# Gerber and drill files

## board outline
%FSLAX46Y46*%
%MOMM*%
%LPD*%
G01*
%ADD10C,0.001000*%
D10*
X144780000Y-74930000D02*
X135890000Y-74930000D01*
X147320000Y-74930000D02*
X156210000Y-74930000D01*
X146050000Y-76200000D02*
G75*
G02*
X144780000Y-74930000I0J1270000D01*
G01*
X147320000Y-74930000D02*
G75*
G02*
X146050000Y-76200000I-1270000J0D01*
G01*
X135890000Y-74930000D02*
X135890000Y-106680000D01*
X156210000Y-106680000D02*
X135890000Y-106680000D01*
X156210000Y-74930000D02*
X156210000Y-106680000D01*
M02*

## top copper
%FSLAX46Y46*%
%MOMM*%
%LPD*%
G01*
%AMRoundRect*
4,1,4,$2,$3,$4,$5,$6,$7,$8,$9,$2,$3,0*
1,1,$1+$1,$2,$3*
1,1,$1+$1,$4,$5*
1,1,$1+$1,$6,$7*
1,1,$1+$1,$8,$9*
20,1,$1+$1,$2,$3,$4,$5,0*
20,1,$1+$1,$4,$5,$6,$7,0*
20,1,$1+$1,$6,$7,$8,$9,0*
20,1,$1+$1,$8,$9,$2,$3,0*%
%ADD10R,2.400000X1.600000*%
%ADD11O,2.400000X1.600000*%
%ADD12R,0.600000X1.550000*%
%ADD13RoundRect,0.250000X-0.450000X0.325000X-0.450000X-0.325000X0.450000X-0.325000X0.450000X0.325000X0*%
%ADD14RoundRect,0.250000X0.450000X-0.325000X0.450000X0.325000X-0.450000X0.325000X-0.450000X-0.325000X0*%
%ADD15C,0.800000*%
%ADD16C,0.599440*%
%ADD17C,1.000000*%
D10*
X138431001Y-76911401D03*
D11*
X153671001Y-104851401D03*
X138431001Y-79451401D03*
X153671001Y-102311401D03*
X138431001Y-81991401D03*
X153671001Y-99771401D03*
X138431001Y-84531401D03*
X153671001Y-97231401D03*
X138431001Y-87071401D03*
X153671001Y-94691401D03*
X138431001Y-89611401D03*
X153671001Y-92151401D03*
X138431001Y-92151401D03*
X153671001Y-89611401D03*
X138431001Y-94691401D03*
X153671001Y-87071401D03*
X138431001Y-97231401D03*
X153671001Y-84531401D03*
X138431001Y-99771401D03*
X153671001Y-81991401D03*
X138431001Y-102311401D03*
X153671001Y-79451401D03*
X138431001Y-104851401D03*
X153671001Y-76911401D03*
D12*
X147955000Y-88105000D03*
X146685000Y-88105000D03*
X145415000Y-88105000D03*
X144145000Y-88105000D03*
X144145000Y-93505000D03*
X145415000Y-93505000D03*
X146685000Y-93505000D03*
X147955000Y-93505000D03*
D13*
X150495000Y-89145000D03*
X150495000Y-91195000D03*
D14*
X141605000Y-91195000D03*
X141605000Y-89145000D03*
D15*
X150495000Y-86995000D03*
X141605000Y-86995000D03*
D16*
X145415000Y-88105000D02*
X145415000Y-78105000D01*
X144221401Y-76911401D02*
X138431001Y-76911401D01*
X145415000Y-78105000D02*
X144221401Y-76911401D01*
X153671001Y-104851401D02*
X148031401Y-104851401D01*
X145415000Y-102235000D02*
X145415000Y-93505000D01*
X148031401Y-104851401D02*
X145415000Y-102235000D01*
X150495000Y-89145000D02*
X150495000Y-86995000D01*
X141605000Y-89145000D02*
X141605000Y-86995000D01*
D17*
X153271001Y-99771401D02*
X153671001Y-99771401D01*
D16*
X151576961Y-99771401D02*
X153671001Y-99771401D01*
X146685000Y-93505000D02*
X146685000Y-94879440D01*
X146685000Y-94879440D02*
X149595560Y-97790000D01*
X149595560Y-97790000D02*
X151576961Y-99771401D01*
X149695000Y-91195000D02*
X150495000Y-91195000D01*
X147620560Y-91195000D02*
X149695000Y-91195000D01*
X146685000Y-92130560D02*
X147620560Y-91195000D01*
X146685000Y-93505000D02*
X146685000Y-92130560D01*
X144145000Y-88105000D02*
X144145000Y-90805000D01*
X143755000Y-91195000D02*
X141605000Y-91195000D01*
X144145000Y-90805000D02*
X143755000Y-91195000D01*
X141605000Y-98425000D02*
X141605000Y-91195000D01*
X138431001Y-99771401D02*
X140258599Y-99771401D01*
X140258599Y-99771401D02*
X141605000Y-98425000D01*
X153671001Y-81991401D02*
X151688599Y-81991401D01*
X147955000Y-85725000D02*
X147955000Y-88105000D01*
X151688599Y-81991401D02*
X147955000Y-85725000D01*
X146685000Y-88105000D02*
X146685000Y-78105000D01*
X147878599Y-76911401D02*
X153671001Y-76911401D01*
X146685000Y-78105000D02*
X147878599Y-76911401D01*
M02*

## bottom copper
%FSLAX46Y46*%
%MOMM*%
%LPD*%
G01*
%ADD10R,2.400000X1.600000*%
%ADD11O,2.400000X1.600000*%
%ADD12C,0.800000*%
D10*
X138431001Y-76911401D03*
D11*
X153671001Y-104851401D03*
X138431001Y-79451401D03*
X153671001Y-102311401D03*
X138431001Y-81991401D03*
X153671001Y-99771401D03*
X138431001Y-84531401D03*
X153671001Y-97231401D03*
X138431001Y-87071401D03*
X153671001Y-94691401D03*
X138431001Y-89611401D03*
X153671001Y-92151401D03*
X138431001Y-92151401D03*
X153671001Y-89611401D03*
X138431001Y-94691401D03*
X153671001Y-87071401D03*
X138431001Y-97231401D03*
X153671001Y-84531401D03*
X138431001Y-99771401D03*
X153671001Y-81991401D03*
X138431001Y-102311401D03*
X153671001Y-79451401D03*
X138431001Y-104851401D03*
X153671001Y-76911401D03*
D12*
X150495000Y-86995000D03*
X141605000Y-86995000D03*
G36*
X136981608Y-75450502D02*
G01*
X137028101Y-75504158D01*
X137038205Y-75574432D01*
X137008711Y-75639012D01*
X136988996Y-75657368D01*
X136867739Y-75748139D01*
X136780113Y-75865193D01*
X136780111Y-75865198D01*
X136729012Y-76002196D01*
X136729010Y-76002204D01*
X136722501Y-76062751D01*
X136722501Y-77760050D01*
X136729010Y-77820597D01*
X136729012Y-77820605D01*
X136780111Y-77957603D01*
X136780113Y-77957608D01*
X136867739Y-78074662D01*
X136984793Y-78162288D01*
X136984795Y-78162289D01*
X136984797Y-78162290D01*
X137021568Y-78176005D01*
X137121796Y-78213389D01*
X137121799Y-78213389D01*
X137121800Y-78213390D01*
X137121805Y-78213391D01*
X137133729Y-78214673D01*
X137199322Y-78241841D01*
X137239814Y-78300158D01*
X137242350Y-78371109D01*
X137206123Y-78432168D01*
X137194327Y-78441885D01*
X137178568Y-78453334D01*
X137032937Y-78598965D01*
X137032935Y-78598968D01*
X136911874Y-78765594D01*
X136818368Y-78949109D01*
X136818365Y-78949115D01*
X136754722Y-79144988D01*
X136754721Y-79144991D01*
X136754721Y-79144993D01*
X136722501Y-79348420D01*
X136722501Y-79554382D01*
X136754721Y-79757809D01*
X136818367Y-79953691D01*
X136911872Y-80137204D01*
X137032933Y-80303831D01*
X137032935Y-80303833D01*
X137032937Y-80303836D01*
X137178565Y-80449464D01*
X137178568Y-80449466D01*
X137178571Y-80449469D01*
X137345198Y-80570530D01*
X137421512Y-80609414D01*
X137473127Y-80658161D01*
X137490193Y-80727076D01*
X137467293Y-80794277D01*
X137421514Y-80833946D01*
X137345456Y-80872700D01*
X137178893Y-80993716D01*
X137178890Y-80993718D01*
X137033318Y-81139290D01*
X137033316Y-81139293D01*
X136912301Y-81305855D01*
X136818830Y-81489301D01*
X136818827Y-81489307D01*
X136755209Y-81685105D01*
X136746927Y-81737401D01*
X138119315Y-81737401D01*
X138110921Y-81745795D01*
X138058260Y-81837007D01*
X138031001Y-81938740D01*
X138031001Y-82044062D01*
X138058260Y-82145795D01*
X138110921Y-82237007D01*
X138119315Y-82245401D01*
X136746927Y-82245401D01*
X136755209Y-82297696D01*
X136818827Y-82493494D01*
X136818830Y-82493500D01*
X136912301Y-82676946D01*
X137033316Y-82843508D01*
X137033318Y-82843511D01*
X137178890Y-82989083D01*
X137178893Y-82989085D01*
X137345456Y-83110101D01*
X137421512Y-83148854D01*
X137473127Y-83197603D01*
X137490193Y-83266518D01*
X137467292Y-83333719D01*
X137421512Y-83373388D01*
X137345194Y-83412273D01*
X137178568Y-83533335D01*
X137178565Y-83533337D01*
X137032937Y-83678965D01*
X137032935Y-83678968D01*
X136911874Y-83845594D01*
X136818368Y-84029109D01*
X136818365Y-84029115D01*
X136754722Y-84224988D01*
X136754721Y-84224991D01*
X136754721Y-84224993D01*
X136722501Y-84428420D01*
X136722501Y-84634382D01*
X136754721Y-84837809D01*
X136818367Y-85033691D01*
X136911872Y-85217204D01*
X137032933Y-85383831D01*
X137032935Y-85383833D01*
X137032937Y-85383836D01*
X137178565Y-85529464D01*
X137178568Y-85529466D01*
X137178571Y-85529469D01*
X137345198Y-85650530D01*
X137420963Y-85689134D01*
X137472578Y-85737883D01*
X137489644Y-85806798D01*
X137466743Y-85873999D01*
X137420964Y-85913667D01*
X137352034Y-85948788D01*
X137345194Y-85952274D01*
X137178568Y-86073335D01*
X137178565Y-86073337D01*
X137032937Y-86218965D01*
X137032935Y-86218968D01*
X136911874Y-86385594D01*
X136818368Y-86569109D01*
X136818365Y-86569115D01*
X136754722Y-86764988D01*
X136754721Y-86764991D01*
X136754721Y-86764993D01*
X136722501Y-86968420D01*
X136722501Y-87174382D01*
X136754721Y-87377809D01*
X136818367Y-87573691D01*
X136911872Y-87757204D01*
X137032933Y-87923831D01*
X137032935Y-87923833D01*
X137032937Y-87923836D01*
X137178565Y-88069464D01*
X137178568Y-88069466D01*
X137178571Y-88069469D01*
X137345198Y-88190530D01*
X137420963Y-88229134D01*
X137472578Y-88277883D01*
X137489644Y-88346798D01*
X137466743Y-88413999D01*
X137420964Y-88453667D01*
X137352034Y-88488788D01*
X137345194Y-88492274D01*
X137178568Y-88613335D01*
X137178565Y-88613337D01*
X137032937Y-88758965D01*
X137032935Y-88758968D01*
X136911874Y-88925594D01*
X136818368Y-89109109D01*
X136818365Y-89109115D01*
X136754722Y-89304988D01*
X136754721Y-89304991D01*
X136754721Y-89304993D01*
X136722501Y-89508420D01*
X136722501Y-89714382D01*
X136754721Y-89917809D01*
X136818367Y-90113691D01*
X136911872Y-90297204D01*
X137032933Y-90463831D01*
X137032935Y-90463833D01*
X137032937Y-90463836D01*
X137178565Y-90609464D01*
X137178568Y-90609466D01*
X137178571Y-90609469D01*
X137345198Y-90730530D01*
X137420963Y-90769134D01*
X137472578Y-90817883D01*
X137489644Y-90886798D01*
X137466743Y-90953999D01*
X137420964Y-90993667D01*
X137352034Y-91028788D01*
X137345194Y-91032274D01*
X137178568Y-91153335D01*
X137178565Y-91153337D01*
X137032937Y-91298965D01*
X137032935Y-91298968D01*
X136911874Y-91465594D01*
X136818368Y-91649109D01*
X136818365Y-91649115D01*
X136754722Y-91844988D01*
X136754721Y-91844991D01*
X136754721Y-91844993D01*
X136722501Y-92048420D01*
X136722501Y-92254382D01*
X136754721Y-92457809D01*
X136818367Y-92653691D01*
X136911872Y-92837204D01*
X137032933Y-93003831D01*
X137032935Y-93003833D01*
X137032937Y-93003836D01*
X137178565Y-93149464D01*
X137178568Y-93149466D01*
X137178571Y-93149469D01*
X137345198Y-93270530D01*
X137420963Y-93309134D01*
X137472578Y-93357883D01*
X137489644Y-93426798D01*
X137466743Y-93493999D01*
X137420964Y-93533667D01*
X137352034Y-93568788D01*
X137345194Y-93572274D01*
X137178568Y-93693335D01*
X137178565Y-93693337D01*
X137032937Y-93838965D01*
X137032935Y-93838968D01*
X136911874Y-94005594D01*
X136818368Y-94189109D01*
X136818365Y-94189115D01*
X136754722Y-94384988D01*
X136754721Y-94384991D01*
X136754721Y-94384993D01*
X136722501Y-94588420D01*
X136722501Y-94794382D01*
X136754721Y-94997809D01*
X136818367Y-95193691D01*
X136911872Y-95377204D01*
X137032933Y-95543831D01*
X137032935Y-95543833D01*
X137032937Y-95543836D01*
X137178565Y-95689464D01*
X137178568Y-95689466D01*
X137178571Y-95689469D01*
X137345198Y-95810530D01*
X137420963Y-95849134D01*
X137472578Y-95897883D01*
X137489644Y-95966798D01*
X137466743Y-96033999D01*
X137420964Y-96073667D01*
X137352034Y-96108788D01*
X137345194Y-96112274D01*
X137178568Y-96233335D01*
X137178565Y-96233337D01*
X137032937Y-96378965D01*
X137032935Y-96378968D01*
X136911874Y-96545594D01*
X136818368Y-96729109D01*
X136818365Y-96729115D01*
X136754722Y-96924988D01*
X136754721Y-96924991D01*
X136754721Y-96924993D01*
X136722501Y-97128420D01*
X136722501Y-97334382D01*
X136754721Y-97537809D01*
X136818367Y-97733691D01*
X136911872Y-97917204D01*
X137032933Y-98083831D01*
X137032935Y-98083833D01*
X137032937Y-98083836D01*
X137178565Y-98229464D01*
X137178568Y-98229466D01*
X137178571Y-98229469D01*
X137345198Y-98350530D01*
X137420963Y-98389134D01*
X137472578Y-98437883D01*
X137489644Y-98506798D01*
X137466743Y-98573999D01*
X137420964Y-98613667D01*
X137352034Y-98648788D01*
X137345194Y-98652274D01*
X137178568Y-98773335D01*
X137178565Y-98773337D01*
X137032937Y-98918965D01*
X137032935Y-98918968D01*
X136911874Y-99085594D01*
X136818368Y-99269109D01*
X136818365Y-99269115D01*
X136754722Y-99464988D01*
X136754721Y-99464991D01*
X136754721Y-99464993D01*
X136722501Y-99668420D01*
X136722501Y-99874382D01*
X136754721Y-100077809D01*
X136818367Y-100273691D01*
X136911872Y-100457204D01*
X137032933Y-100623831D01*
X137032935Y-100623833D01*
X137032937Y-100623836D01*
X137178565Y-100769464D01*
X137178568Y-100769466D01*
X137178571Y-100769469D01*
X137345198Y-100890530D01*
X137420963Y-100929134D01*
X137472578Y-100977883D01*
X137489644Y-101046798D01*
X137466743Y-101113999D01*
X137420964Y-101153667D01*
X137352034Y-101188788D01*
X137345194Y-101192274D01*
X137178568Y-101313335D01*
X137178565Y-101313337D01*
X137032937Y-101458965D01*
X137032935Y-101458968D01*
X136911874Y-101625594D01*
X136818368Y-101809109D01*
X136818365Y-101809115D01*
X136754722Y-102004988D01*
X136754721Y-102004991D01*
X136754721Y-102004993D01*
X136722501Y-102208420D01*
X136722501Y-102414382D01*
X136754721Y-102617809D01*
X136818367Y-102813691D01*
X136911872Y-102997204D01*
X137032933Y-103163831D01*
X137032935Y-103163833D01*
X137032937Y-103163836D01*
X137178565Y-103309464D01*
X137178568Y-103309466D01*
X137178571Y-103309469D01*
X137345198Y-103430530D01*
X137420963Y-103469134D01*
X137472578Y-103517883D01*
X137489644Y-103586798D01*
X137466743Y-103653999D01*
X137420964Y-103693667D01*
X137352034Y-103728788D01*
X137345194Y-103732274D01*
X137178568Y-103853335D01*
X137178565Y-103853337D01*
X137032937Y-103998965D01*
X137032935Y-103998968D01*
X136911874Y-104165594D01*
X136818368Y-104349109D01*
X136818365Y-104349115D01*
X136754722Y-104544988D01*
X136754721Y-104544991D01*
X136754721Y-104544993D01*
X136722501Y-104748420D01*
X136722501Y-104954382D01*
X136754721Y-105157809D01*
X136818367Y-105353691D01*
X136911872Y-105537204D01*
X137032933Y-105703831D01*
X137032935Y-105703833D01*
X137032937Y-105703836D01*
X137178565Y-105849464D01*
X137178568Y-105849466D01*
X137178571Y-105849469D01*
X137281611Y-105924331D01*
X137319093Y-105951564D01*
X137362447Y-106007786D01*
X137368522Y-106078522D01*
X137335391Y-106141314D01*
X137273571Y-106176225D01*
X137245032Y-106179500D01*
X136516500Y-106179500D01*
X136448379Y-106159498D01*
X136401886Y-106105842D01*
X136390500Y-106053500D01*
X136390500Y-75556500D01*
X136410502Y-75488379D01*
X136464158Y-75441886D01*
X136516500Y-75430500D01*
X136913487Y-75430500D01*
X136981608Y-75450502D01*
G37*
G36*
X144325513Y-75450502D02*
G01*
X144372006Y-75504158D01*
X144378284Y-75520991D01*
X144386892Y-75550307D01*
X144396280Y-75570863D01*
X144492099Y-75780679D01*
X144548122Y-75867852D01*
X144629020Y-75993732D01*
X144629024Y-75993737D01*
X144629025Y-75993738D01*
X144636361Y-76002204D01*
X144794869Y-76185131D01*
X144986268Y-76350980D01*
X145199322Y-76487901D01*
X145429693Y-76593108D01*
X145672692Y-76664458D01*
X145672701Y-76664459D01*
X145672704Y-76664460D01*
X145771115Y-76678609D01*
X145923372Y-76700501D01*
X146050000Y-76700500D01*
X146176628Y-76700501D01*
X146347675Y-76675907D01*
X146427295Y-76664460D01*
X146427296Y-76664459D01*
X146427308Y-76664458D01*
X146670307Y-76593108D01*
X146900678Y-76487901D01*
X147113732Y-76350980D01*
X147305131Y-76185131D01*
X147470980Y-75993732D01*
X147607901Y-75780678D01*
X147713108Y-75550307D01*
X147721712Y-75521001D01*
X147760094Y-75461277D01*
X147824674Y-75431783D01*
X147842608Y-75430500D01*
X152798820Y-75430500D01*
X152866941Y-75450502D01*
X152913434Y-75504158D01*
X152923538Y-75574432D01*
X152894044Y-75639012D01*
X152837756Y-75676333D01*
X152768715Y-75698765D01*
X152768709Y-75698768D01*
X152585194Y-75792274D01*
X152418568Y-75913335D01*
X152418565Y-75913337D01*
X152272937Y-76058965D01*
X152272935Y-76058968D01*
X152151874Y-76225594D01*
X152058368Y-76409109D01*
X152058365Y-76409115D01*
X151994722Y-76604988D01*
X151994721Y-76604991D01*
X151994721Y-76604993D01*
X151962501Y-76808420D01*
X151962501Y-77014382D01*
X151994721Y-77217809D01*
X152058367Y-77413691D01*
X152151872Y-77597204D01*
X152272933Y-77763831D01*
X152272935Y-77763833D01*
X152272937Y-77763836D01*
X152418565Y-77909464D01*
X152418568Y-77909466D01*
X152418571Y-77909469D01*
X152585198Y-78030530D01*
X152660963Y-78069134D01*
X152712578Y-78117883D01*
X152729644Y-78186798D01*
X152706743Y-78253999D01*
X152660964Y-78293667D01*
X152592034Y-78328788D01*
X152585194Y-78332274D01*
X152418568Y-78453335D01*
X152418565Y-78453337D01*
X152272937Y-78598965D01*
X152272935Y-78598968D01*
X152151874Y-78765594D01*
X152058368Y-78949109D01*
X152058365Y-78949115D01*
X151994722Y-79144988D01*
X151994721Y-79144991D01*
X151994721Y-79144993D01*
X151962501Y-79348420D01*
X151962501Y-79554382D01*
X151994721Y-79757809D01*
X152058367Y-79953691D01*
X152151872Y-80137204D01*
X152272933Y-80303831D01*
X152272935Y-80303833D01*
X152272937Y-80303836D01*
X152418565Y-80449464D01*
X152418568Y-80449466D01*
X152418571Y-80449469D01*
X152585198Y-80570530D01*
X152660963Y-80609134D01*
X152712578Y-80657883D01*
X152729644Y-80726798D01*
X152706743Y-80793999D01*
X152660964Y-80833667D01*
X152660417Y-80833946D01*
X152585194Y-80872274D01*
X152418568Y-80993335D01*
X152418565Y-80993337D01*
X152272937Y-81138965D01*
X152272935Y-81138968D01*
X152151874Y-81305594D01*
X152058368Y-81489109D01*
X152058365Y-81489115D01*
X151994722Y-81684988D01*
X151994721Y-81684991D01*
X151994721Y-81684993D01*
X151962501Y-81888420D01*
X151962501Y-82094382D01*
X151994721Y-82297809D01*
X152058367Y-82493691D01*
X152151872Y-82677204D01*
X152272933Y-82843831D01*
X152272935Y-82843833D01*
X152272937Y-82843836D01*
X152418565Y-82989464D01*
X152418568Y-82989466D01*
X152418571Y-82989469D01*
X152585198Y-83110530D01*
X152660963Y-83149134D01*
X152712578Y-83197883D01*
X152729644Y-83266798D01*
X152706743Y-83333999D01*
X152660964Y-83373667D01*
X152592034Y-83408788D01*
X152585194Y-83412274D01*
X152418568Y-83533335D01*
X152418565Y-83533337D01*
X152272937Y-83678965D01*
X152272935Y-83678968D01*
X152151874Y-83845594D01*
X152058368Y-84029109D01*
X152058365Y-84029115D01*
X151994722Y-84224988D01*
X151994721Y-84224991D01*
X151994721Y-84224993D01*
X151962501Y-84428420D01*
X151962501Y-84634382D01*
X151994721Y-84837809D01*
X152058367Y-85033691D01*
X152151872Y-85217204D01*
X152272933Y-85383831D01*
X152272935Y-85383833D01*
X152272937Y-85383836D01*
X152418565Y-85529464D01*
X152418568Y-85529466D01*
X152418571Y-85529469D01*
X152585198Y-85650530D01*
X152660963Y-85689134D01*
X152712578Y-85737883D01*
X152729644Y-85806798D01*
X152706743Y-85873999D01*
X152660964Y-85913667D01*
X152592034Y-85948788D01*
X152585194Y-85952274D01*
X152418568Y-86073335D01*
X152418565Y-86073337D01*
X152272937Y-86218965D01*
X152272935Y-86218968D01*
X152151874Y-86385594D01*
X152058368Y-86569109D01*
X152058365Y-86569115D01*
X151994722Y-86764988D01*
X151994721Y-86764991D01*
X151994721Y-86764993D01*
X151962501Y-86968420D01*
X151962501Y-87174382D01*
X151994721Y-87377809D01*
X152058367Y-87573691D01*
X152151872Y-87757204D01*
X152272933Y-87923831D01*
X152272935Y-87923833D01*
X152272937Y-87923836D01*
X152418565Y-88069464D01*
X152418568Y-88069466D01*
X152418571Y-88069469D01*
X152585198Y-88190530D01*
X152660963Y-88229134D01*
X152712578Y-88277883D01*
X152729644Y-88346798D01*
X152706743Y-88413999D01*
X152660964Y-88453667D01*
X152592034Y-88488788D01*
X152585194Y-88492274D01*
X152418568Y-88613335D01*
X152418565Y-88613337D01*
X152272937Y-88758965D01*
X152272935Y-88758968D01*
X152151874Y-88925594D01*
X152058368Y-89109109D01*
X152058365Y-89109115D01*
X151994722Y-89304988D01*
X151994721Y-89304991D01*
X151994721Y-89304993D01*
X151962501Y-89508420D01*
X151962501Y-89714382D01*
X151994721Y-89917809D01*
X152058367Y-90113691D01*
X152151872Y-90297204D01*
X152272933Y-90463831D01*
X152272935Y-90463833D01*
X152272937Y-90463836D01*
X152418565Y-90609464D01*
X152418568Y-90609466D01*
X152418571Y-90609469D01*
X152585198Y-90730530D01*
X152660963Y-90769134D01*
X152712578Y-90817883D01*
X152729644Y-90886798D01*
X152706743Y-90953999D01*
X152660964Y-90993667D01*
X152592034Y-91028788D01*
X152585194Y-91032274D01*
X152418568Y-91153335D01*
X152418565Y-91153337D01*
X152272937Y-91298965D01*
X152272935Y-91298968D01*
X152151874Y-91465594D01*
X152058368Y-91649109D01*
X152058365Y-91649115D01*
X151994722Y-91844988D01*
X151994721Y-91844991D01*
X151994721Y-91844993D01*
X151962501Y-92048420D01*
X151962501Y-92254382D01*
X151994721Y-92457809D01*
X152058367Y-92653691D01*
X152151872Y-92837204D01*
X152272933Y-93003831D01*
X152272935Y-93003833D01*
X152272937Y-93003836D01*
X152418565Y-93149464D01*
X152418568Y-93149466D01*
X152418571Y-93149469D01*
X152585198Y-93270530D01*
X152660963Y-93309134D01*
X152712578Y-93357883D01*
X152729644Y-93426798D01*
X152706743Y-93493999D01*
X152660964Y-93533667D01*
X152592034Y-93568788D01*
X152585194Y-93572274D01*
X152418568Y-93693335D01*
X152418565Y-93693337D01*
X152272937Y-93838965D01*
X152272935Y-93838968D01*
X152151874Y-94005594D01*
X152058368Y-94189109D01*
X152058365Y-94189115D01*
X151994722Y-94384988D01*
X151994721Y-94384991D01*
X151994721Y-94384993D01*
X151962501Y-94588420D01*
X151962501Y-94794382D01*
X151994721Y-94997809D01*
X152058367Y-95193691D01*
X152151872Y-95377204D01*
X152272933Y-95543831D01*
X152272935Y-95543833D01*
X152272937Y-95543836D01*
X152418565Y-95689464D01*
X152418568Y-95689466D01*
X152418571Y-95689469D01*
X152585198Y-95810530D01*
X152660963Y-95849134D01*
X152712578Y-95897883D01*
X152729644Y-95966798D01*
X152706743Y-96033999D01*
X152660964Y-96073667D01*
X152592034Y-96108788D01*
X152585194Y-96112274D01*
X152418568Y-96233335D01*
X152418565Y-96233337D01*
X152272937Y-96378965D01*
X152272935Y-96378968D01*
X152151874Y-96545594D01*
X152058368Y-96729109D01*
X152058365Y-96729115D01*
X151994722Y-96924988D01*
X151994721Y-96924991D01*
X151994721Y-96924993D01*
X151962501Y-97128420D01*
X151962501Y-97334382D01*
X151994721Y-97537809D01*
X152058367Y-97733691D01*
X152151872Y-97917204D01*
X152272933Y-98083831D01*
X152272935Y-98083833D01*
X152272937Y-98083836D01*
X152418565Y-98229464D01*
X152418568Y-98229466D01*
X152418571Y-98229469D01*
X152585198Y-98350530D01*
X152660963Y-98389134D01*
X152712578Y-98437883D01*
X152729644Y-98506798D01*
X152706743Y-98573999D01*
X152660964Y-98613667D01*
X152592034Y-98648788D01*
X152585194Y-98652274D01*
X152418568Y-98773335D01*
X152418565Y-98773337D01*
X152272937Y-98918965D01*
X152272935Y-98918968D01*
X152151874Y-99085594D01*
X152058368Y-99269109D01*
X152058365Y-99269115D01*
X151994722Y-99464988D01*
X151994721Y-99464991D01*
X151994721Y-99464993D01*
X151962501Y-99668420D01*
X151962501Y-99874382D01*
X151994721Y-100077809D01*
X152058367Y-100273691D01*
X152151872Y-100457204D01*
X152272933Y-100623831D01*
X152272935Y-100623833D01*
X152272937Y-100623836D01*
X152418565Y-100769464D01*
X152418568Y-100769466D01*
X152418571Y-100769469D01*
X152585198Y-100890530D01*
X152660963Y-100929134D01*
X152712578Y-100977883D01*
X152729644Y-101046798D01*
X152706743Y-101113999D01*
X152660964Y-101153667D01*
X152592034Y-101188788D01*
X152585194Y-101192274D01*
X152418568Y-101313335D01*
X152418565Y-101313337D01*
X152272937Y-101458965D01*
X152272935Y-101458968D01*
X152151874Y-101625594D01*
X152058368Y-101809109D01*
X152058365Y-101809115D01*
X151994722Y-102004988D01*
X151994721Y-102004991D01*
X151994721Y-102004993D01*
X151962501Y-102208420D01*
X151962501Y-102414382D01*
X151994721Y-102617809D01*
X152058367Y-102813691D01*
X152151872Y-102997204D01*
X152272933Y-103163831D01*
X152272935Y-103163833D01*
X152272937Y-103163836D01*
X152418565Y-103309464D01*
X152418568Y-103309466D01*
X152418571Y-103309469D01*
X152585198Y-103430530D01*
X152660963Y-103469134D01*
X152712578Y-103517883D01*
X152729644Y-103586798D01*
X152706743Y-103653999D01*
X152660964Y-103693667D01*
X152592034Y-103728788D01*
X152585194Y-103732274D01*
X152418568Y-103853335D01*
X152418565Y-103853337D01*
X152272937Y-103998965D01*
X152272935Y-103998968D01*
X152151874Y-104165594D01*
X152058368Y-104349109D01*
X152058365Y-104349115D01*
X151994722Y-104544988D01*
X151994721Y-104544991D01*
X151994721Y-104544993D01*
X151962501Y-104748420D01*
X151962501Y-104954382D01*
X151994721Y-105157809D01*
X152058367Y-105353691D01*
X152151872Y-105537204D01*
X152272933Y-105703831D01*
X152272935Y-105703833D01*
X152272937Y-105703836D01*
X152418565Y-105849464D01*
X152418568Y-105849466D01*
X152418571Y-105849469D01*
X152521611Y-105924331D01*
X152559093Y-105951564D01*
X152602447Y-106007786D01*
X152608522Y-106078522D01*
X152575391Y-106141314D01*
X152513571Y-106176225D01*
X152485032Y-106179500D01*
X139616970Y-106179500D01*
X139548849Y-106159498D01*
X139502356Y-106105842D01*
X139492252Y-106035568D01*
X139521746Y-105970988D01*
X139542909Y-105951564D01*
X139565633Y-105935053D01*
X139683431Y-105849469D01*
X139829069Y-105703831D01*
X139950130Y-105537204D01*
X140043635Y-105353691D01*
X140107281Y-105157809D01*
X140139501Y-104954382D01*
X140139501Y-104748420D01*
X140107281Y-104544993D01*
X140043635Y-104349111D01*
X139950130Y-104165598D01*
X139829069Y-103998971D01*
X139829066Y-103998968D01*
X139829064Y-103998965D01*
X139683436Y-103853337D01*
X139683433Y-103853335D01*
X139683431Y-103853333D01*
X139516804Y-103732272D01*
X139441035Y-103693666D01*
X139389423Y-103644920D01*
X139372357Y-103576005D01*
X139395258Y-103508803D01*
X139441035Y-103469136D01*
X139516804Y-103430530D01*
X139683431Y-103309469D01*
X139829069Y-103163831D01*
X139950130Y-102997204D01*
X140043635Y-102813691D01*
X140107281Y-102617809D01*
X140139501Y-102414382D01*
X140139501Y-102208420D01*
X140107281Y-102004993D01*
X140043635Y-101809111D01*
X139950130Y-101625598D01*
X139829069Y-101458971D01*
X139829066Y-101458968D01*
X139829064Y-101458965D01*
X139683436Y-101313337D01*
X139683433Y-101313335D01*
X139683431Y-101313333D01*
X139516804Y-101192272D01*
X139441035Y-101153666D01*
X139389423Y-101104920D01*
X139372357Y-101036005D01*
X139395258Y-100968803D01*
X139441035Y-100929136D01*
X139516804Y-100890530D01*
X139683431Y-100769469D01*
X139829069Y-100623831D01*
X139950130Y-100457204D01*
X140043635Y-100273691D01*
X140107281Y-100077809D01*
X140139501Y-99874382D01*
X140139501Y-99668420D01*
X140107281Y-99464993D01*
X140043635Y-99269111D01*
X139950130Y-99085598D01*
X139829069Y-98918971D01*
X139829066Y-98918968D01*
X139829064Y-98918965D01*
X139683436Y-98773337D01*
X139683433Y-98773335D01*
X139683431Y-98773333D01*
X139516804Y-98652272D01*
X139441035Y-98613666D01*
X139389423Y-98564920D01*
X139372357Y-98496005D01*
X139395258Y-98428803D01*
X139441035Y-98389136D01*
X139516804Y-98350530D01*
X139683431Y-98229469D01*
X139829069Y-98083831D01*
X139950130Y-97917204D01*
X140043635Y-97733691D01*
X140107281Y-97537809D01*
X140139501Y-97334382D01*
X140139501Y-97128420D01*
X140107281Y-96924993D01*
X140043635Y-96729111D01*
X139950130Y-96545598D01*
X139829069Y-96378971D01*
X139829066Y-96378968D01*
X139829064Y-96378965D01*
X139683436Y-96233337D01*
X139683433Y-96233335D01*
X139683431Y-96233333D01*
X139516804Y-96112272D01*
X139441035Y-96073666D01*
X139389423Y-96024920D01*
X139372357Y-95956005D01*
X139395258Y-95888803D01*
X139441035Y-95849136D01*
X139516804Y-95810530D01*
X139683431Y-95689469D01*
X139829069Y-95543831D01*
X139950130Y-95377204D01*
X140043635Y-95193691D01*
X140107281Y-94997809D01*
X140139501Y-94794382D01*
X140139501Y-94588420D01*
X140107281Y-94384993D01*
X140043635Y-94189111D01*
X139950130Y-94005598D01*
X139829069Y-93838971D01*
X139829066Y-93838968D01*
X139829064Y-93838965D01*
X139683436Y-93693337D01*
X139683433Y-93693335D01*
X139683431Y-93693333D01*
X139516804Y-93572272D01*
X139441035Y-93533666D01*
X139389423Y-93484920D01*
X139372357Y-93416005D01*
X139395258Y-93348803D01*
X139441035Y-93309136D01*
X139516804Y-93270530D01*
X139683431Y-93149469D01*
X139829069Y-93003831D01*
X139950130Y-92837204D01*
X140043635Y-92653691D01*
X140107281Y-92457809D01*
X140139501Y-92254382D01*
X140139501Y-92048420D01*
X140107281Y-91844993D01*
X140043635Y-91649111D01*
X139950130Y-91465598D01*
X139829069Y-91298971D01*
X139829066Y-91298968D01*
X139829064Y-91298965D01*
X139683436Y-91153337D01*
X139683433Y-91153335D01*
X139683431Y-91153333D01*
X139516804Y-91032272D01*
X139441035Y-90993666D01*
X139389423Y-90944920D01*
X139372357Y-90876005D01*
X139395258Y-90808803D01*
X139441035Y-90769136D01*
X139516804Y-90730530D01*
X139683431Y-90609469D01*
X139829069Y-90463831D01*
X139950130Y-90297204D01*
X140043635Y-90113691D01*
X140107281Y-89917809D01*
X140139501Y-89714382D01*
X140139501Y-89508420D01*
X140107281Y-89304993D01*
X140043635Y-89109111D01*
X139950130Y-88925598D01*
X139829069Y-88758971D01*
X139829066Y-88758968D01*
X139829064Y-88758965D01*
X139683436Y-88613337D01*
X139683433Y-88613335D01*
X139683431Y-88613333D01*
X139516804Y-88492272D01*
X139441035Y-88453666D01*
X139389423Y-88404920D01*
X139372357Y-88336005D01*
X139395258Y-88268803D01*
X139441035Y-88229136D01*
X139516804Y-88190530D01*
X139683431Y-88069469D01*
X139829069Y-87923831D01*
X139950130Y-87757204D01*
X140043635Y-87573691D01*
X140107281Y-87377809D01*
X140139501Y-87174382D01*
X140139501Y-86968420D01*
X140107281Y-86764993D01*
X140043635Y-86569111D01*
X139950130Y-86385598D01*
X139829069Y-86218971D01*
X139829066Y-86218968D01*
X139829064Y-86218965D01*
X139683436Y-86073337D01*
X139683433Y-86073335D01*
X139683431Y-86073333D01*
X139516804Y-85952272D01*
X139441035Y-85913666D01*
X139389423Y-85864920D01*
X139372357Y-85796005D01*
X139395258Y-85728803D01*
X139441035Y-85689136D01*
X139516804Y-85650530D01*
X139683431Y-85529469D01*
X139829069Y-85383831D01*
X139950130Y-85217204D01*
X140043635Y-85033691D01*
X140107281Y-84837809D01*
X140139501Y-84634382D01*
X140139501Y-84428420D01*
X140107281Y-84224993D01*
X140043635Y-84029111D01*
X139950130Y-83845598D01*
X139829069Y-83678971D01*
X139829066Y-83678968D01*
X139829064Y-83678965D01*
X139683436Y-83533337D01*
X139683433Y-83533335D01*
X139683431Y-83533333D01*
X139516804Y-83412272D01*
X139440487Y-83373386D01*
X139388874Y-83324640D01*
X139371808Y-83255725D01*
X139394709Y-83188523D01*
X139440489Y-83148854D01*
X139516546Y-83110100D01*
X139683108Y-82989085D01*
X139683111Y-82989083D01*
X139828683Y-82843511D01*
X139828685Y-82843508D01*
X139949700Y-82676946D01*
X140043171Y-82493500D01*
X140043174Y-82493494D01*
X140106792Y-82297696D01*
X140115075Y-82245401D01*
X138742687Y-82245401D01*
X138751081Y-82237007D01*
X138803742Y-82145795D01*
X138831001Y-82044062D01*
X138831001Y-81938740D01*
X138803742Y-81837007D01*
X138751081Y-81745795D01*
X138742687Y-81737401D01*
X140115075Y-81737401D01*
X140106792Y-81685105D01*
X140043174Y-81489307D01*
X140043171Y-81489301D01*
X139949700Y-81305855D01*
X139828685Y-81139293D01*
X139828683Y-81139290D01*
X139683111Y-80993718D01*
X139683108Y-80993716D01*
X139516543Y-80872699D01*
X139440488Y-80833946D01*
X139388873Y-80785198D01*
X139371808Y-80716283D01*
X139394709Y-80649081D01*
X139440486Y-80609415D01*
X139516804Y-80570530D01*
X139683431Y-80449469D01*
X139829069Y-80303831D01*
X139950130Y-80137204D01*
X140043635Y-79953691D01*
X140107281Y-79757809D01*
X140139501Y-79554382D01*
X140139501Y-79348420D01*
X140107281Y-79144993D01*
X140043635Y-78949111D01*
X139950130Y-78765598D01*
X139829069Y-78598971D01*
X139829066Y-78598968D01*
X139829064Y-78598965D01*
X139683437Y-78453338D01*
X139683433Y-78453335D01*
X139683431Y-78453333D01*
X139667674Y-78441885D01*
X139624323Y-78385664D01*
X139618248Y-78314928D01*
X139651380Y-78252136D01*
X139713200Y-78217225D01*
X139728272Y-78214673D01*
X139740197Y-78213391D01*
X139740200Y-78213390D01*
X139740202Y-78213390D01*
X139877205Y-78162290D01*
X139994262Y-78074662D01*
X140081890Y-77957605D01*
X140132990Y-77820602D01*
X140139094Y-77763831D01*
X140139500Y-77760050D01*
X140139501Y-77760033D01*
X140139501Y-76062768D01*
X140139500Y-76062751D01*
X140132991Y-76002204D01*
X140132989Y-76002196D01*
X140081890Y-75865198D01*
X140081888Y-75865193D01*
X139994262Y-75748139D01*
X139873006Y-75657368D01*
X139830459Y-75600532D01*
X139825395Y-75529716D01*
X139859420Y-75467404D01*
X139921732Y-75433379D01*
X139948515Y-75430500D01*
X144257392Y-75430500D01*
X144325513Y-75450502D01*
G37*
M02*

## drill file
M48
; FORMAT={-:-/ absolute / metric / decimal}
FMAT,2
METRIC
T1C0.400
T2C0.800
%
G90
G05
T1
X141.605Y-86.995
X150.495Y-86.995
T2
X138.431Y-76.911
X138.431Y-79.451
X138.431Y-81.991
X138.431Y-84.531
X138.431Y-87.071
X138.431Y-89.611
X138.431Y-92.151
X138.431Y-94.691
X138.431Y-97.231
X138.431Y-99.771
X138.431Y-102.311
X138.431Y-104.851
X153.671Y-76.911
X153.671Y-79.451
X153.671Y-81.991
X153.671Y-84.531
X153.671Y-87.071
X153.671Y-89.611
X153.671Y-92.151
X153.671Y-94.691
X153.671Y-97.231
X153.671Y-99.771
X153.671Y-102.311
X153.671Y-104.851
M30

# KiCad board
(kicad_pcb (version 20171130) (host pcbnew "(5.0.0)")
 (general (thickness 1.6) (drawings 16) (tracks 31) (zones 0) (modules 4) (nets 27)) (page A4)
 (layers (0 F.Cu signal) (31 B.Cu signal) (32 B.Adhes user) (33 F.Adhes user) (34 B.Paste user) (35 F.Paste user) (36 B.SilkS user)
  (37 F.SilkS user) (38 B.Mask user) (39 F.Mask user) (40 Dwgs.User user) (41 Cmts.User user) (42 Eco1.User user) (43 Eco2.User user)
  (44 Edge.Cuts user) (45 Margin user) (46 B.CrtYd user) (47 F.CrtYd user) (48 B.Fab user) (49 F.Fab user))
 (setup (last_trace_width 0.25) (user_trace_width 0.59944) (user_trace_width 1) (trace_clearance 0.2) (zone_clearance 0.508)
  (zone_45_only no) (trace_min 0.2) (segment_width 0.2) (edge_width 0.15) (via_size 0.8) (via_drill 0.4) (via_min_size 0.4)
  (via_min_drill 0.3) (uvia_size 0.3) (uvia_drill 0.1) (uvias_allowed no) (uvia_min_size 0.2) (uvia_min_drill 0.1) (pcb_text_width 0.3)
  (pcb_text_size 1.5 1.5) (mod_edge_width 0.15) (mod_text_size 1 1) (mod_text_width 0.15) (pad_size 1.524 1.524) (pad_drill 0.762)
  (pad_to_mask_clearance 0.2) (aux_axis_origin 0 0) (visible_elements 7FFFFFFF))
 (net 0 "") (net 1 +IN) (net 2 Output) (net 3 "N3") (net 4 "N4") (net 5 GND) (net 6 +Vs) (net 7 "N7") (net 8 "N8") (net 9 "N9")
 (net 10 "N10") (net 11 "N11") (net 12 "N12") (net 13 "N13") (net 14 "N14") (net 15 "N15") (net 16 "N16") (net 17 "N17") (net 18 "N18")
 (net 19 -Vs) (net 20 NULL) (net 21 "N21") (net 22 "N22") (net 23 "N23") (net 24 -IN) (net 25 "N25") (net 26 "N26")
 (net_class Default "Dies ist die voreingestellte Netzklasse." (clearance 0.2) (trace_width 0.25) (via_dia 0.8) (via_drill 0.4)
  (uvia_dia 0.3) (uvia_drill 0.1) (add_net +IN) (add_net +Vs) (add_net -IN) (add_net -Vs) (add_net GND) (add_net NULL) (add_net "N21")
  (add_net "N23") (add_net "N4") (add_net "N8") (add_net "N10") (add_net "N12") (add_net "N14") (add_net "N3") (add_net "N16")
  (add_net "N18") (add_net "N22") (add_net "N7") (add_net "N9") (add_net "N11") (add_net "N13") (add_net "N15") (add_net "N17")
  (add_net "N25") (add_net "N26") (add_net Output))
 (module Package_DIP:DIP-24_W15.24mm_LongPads (layer F.Cu) (at 138.431001 76.911401)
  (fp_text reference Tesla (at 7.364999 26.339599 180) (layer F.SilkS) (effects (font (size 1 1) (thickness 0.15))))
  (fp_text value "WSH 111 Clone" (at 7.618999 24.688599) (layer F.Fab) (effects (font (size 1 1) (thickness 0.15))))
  (pad 1 thru_hole rect (at 0 0) (size 2.4 1.6) (drill 0.8) (layers *.Cu *.Mask) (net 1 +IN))
  (pad 13 thru_hole oval (at 15.24 27.94) (size 2.4 1.6) (drill 0.8) (layers *.Cu *.Mask) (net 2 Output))
  (pad 2 thru_hole oval (at 0 2.54) (size 2.4 1.6) (drill 0.8) (layers *.Cu *.Mask) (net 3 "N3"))
  (pad 14 thru_hole oval (at 15.24 25.4) (size 2.4 1.6) (drill 0.8) (layers *.Cu *.Mask) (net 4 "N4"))
  (pad 3 thru_hole oval (at 0 5.08) (size 2.4 1.6) (drill 0.8) (layers *.Cu *.Mask) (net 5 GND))
  (pad 15 thru_hole oval (at 15.24 22.86) (size 2.4 1.6) (drill 0.8) (layers *.Cu *.Mask) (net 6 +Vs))
  (pad 4 thru_hole oval (at 0 7.62) (size 2.4 1.6) (drill 0.8) (layers *.Cu *.Mask) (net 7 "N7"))
  (pad 16 thru_hole oval (at 15.24 20.32) (size 2.4 1.6) (drill 0.8) (layers *.Cu *.Mask) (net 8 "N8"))
  (pad 5 thru_hole oval (at 0 10.16) (size 2.4 1.6) (drill 0.8) (layers *.Cu *.Mask) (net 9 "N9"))
  (pad 17 thru_hole oval (at 15.24 17.78) (size 2.4 1.6) (drill 0.8) (layers *.Cu *.Mask) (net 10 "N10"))
  (pad 6 thru_hole oval (at 0 12.7) (size 2.4 1.6) (drill 0.8) (layers *.Cu *.Mask) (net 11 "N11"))
  (pad 18 thru_hole oval (at 15.24 15.24) (size 2.4 1.6) (drill 0.8) (layers *.Cu *.Mask) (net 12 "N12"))
  (pad 7 thru_hole oval (at 0 15.24) (size 2.4 1.6) (drill 0.8) (layers *.Cu *.Mask) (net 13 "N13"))
  (pad 19 thru_hole oval (at 15.24 12.7) (size 2.4 1.6) (drill 0.8) (layers *.Cu *.Mask) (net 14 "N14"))
  (pad 8 thru_hole oval (at 0 17.78) (size 2.4 1.6) (drill 0.8) (layers *.Cu *.Mask) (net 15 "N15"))
  (pad 20 thru_hole oval (at 15.24 10.16) (size 2.4 1.6) (drill 0.8) (layers *.Cu *.Mask) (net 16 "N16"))
  (pad 9 thru_hole oval (at 0 20.32) (size 2.4 1.6) (drill 0.8) (layers *.Cu *.Mask) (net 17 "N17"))
  (pad 21 thru_hole oval (at 15.24 7.62) (size 2.4 1.6) (drill 0.8) (layers *.Cu *.Mask) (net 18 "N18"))
  (pad 10 thru_hole oval (at 0 22.86) (size 2.4 1.6) (drill 0.8) (layers *.Cu *.Mask) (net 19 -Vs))
  (pad 22 thru_hole oval (at 15.24 5.08) (size 2.4 1.6) (drill 0.8) (layers *.Cu *.Mask) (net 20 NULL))
  (pad 11 thru_hole oval (at 0 25.4) (size 2.4 1.6) (drill 0.8) (layers *.Cu *.Mask) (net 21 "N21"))
  (pad 23 thru_hole oval (at 15.24 2.54) (size 2.4 1.6) (drill 0.8) (layers *.Cu *.Mask) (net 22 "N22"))
  (pad 12 thru_hole oval (at 0 27.94) (size 2.4 1.6) (drill 0.8) (layers *.Cu *.Mask) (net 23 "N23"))
  (pad 24 thru_hole oval (at 15.24 0) (size 2.4 1.6) (drill 0.8) (layers *.Cu *.Mask) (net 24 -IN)))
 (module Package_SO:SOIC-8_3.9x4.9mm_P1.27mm (layer F.Cu) (at 146.05 90.805 270)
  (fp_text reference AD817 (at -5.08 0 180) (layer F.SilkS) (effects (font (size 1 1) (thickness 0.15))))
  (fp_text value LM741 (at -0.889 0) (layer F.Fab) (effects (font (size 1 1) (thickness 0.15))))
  (pad 1 smd rect (at -2.7 -1.905 270) (size 1.55 0.6) (layers F.Cu F.Paste F.Mask) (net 20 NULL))
  (pad 2 smd rect (at -2.7 -0.635 270) (size 1.55 0.6) (layers F.Cu F.Paste F.Mask) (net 24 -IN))
  (pad 3 smd rect (at -2.7 0.635 270) (size 1.55 0.6) (layers F.Cu F.Paste F.Mask) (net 1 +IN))
  (pad 4 smd rect (at -2.7 1.905 270) (size 1.55 0.6) (layers F.Cu F.Paste F.Mask) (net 19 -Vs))
  (pad 5 smd rect (at 2.7 1.905 270) (size 1.55 0.6) (layers F.Cu F.Paste F.Mask) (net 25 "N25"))
  (pad 6 smd rect (at 2.7 0.635 270) (size 1.55 0.6) (layers F.Cu F.Paste F.Mask) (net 2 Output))
  (pad 7 smd rect (at 2.7 -0.635 270) (size 1.55 0.6) (layers F.Cu F.Paste F.Mask) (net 6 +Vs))
  (pad 8 smd rect (at 2.7 -1.905 270) (size 1.55 0.6) (layers F.Cu F.Paste F.Mask) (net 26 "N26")))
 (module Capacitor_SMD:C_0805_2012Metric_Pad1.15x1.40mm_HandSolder (layer F.Cu) (at 150.495 90.17 270)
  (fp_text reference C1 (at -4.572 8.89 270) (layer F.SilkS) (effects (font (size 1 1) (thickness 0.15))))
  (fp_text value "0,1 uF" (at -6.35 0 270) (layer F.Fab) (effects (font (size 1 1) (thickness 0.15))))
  (pad 1 smd roundrect (at -1.025 0 270) (size 1.15 1.4) (layers F.Cu F.Paste F.Mask) (roundrect_rratio 0.217391) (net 5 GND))
  (pad 2 smd roundrect (at 1.025 0 270) (size 1.15 1.4) (layers F.Cu F.Paste F.Mask) (roundrect_rratio 0.217391) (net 6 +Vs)))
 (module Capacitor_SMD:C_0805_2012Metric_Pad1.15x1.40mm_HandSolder (layer F.Cu) (at 141.605 90.17 90)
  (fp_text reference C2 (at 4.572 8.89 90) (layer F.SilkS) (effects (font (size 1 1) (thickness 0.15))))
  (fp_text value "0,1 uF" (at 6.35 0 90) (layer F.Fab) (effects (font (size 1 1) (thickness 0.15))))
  (pad 1 smd roundrect (at -1.025 0 90) (size 1.15 1.4) (layers F.Cu F.Paste F.Mask) (roundrect_rratio 0.217391) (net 19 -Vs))
  (pad 2 smd roundrect (at 1.025 0 90) (size 1.15 1.4) (layers F.Cu F.Paste F.Mask) (roundrect_rratio 0.217391) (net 5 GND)))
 (gr_line (start 144.78 74.93) (end 135.89 74.93) (layer Edge.Cuts) (width 0.001))
 (gr_line (start 147.32 74.93) (end 156.21 74.93) (layer Edge.Cuts) (width 0.001))
 (gr_arc (start 146.05 74.93) (end 144.78 74.93) (angle -90) (layer Edge.Cuts) (width 0.001))
 (gr_arc (start 146.05 74.93) (end 146.05 76.2) (angle -90) (layer Edge.Cuts) (width 0.001))
 (gr_line (start 135.89 74.93) (end 135.89 106.68) (layer Edge.Cuts) (width 0.001))
 (gr_line (start 156.21 106.68) (end 135.89 106.68) (layer Edge.Cuts) (width 0.001))
 (gr_line (start 156.21 74.93) (end 156.21 106.68) (layer Edge.Cuts) (width 0.001))
 (segment (start 145.415 88.105) (end 145.415 78.105) (width 0.59944) (layer F.Cu) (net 1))
 (segment (start 144.221401 76.911401) (end 138.431001 76.911401) (width 0.59944) (layer F.Cu) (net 1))
 (segment (start 145.415 78.105) (end 144.221401 76.911401) (width 0.59944) (layer F.Cu) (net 1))
 (segment (start 153.671001 104.851401) (end 148.031401 104.851401) (width 0.59944) (layer F.Cu) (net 2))
 (segment (start 145.415 102.235) (end 145.415 93.505) (width 0.59944) (layer F.Cu) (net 2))
 (segment (start 148.031401 104.851401) (end 145.415 102.235) (width 0.59944) (layer F.Cu) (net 2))
 (segment (start 150.495 89.145) (end 150.495 86.995) (width 0.59944) (layer F.Cu) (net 5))
 (via (at 150.495 86.995) (size 0.8) (drill 0.4) (layers F.Cu B.Cu) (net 5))
 (segment (start 141.605 89.145) (end 141.605 86.995) (width 0.59944) (layer F.Cu) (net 5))
 (via (at 141.605 86.995) (size 0.8) (drill 0.4) (layers F.Cu B.Cu) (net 5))
 (segment (start 153.271001 99.771401) (end 153.671001 99.771401) (width 1) (layer F.Cu) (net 6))
 (segment (start 151.576961 99.771401) (end 153.671001 99.771401) (width 0.59944) (layer F.Cu) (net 6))
 (segment (start 146.685 93.505) (end 146.685 94.87944) (width 0.59944) (layer F.Cu) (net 6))
 (segment (start 146.685 94.87944) (end 149.59556 97.79) (width 0.59944) (layer F.Cu) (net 6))
 (segment (start 149.59556 97.79) (end 151.576961 99.771401) (width 0.59944) (layer F.Cu) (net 6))
 (segment (start 149.695 91.195) (end 150.495 91.195) (width 0.59944) (layer F.Cu) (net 6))
 (segment (start 147.62056 91.195) (end 149.695 91.195) (width 0.59944) (layer F.Cu) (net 6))
 (segment (start 146.685 92.13056) (end 147.62056 91.195) (width 0.59944) (layer F.Cu) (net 6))
 (segment (start 146.685 93.505) (end 146.685 92.13056) (width 0.59944) (layer F.Cu) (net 6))
 (segment (start 144.145 88.105) (end 144.145 90.805) (width 0.59944) (layer F.Cu) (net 19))
 (segment (start 143.755 91.195) (end 141.605 91.195) (width 0.59944) (layer F.Cu) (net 19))
 (segment (start 144.145 90.805) (end 143.755 91.195) (width 0.59944) (layer F.Cu) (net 19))
 (segment (start 141.605 98.425) (end 141.605 91.195) (width 0.59944) (layer F.Cu) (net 19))
 (segment (start 138.431001 99.771401) (end 140.258599 99.771401) (width 0.59944) (layer F.Cu) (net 19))
 (segment (start 140.258599 99.771401) (end 141.605 98.425) (width 0.59944) (layer F.Cu) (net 19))
 (segment (start 153.671001 81.991401) (end 151.688599 81.991401) (width 0.59944) (layer F.Cu) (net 20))
 (segment (start 147.955 85.725) (end 147.955 88.105) (width 0.59944) (layer F.Cu) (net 20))
 (segment (start 151.688599 81.991401) (end 147.955 85.725) (width 0.59944) (layer F.Cu) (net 20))
 (segment (start 146.685 88.105) (end 146.685 78.105) (width 0.59944) (layer F.Cu) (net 24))
 (segment (start 147.878599 76.911401) (end 153.671001 76.911401) (width 0.59944) (layer F.Cu) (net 24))
 (segment (start 146.685 78.105) (end 147.878599 76.911401) (width 0.59944) (layer F.Cu) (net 24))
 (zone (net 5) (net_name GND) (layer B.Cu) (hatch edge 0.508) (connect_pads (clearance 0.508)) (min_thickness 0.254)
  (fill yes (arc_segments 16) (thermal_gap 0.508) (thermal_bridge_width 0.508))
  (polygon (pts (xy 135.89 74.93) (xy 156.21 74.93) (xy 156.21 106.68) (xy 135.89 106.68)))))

